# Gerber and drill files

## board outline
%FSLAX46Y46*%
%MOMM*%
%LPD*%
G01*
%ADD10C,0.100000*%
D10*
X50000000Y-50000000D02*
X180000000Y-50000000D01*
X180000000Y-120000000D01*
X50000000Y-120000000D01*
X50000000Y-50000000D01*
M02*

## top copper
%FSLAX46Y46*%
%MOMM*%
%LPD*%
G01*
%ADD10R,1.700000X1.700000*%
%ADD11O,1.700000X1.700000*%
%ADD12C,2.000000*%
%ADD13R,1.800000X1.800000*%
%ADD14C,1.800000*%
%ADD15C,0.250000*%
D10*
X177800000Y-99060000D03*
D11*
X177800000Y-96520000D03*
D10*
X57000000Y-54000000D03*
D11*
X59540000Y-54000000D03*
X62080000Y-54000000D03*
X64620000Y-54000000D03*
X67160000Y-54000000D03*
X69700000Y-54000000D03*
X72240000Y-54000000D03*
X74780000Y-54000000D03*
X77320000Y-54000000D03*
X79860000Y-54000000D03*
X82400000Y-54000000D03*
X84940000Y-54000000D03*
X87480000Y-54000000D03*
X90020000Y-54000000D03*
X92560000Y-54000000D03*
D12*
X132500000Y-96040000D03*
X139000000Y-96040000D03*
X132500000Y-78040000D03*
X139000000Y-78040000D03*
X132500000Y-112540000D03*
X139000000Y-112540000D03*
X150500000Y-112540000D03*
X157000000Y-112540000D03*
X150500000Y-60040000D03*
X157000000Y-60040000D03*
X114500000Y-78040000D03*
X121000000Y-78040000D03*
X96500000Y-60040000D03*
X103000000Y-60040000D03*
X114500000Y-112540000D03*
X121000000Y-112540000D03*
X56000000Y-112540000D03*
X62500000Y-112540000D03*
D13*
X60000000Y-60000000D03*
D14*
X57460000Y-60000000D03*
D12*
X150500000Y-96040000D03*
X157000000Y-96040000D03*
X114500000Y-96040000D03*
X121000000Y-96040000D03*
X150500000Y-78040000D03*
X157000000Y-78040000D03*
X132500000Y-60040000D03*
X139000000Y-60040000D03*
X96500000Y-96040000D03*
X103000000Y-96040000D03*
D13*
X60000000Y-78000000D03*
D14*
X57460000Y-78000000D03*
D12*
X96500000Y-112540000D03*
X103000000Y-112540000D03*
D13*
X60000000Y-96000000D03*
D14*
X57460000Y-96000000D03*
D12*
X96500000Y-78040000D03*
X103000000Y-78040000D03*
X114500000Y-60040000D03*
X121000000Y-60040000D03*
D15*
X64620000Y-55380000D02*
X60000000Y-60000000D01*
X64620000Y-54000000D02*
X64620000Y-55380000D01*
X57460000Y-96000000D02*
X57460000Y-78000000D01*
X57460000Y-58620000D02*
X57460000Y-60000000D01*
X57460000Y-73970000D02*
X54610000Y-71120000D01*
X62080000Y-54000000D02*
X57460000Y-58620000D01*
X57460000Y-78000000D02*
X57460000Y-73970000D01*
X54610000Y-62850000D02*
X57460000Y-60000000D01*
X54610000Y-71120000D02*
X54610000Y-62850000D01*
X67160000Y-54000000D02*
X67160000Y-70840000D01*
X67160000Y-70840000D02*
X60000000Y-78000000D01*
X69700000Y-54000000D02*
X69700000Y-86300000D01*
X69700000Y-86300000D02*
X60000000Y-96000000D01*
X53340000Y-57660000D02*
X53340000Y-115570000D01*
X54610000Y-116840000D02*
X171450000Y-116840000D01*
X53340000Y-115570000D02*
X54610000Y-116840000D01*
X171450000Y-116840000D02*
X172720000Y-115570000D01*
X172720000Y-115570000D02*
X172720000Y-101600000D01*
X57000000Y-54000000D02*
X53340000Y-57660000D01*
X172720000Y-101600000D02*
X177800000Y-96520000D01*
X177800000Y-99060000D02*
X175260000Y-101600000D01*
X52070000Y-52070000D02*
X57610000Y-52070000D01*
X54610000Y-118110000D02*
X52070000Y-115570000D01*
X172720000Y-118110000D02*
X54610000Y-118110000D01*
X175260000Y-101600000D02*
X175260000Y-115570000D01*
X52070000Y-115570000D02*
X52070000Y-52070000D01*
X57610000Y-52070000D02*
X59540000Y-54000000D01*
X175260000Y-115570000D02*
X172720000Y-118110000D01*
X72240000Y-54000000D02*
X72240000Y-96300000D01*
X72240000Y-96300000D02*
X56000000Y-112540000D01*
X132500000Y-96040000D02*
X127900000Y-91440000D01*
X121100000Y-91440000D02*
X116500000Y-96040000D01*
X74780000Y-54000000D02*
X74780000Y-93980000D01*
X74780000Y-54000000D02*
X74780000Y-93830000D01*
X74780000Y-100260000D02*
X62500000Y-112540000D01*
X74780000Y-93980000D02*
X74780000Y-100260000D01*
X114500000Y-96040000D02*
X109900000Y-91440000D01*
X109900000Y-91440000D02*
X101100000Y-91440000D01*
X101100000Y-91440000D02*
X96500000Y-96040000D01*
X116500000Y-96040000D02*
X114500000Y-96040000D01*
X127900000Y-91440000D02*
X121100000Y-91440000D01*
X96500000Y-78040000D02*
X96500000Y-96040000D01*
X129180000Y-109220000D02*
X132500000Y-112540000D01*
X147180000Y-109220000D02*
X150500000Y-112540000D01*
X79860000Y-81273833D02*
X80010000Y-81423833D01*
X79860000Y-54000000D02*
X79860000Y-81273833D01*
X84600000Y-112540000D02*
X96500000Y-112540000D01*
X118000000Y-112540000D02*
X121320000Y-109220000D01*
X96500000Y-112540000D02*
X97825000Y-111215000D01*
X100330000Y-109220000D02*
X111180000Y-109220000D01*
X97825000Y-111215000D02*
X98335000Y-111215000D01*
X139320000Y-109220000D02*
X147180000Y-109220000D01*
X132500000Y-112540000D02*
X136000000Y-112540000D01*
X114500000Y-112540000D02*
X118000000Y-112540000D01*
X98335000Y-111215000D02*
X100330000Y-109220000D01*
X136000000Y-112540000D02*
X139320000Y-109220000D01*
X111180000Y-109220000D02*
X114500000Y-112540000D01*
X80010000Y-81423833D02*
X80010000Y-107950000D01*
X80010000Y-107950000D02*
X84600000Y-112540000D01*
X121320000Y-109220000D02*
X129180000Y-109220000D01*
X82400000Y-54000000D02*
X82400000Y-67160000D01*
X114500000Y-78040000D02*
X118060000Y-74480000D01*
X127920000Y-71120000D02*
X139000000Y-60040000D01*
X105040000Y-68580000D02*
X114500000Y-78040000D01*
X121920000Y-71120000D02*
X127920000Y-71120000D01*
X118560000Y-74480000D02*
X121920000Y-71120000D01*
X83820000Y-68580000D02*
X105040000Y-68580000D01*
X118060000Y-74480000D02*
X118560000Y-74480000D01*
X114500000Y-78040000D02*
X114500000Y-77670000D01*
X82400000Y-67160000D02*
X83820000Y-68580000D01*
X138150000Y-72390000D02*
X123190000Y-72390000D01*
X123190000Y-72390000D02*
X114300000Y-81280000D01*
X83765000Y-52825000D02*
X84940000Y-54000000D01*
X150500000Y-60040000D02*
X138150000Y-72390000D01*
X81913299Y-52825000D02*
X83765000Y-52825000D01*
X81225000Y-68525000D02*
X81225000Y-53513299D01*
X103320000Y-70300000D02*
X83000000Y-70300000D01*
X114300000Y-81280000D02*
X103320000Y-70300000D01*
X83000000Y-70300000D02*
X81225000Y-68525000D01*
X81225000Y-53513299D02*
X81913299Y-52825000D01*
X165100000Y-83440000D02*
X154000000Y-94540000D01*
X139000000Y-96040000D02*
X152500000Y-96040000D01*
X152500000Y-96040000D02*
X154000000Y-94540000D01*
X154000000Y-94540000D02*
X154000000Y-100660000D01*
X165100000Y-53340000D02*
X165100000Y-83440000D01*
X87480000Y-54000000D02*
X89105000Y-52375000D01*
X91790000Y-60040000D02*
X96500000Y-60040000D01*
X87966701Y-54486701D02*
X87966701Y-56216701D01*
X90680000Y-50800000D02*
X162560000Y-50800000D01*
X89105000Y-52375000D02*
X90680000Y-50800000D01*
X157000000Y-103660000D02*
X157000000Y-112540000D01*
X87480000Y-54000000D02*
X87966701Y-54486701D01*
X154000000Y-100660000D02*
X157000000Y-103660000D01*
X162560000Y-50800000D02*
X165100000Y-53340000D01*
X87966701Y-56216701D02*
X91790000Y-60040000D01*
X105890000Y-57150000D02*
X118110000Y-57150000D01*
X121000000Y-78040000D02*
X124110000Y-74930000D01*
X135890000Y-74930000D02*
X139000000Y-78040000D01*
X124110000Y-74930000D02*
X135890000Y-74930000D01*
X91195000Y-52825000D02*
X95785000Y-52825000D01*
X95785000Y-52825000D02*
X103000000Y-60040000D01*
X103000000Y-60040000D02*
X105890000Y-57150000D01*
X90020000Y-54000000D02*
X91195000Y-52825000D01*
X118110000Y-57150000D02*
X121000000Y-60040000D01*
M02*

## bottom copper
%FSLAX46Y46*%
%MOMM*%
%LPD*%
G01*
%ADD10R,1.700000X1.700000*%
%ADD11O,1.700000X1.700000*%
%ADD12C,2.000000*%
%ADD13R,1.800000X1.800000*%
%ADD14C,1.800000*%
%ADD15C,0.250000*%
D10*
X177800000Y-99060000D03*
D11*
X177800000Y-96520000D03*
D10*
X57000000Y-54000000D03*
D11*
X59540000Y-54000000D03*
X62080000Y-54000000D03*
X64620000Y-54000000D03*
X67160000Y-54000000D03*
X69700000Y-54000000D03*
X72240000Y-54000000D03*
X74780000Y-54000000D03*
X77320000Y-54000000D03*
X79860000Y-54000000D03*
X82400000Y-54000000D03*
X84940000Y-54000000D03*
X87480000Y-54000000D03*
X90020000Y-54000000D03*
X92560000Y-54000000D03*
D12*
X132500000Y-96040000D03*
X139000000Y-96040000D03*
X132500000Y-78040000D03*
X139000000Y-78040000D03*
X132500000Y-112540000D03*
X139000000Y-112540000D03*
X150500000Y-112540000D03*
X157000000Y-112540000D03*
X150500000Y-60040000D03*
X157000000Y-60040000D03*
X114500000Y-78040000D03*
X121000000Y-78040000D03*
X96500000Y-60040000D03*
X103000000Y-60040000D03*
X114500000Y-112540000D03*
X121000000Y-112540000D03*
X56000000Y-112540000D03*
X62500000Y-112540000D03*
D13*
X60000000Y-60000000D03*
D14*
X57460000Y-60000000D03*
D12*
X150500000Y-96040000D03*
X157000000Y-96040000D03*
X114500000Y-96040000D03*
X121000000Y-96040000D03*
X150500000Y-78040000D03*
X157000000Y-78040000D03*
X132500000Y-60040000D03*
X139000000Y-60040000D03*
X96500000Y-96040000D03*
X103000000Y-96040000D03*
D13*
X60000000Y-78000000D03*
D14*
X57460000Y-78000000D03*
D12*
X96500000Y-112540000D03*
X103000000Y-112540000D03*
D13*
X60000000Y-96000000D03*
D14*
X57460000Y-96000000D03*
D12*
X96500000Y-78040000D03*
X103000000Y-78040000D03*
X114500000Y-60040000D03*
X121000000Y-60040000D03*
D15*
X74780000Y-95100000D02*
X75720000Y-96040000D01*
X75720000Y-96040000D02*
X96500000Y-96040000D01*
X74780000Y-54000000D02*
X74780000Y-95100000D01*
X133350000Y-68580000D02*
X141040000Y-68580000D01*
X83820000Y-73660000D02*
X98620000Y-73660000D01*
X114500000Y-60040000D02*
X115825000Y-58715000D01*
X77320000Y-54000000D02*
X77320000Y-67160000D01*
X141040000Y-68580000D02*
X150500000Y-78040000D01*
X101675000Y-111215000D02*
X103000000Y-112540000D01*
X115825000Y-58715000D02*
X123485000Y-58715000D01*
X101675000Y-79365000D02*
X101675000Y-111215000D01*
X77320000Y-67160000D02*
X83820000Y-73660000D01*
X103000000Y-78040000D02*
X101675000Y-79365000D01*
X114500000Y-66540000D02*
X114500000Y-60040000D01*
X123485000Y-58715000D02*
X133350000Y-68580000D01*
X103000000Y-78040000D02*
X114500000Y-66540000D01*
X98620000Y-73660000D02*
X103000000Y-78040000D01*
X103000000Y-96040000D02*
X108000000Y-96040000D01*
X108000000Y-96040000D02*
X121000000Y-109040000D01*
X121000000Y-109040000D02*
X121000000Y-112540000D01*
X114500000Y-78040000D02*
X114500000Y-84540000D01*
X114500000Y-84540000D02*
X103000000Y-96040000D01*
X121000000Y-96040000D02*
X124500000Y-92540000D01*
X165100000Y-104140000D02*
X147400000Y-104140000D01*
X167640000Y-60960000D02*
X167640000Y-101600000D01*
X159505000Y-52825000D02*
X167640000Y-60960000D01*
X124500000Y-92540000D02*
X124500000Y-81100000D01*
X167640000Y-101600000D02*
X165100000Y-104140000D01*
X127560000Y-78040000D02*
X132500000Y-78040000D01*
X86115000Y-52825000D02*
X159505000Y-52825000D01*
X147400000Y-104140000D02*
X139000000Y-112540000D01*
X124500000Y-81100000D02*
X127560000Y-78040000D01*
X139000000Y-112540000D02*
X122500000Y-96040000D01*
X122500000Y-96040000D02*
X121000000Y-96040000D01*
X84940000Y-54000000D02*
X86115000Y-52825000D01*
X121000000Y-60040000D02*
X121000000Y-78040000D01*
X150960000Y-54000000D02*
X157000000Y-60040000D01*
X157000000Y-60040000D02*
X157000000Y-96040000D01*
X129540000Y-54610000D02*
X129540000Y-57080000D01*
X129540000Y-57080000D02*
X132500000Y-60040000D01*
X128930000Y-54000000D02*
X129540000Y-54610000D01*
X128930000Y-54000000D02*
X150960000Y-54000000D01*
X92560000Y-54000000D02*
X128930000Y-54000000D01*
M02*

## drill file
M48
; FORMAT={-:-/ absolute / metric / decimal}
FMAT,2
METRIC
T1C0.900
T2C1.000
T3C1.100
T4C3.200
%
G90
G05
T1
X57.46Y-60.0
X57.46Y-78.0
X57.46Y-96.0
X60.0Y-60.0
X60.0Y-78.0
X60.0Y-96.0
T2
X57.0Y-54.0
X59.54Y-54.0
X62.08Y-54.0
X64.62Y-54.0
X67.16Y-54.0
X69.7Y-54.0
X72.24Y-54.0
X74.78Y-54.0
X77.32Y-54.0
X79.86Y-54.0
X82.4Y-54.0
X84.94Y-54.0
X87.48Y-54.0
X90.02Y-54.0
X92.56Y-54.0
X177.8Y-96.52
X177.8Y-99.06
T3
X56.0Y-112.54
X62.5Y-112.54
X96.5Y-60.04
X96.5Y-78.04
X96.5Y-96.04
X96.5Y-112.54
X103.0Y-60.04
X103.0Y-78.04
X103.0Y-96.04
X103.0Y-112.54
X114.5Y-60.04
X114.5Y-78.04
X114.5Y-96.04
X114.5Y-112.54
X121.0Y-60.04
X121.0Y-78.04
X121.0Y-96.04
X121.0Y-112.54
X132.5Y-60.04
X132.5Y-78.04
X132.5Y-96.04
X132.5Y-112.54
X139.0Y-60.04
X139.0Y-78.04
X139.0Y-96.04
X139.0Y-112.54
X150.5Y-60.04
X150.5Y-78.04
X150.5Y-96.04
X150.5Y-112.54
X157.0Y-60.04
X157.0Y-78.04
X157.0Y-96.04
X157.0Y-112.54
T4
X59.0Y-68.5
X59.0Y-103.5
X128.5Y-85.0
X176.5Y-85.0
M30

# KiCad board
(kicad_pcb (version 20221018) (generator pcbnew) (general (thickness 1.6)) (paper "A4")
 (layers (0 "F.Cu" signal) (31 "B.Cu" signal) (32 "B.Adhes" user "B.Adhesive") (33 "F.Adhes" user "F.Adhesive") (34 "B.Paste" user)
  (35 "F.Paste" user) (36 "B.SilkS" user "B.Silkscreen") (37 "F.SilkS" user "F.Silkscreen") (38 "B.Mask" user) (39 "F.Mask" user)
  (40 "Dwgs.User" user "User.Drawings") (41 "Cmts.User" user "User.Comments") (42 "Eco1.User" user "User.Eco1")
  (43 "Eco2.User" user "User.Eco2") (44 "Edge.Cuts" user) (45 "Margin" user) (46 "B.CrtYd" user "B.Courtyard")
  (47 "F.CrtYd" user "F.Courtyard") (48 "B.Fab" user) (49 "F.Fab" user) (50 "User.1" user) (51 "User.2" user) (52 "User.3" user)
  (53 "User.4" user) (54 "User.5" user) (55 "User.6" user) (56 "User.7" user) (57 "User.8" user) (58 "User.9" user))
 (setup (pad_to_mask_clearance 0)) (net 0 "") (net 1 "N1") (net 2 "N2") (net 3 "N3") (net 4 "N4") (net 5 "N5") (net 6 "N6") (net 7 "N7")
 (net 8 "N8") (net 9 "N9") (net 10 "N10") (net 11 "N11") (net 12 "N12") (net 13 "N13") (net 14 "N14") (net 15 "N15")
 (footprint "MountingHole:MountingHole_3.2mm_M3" (layer "F.Cu") (at 59 68.5)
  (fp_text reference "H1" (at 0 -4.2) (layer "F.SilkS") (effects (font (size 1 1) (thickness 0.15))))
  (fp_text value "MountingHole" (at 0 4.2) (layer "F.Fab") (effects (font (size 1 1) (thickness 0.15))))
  (pad "" np_thru_hole circle (at 0 0) (size 3.2 3.2) (drill 3.2) (layers "*.Cu" "*.Mask")))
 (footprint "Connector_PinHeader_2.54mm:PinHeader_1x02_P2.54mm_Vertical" (layer "F.Cu") (at 177.8 99.06 180)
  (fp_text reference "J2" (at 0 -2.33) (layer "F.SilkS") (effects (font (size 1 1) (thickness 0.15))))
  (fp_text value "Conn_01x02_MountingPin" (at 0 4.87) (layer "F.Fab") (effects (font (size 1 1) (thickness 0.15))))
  (pad "1" thru_hole rect (at 0 0 180) (size 1.7 1.7) (drill 1) (layers "*.Cu" "*.Mask") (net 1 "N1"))
  (pad "2" thru_hole oval (at 0 2.54 180) (size 1.7 1.7) (drill 1) (layers "*.Cu" "*.Mask") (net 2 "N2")))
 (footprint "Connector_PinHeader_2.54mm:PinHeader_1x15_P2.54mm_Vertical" (layer "F.Cu") (at 57 54 90)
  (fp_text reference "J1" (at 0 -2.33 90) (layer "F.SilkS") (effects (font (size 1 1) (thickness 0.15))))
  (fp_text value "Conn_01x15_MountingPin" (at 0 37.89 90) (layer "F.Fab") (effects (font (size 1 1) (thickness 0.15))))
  (pad "1" thru_hole rect (at 0 0 90) (size 1.7 1.7) (drill 1) (layers "*.Cu" "*.Mask") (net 2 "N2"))
  (pad "2" thru_hole oval (at 0 2.54 90) (size 1.7 1.7) (drill 1) (layers "*.Cu" "*.Mask") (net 1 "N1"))
  (pad "3" thru_hole oval (at 0 5.08 90) (size 1.7 1.7) (drill 1) (layers "*.Cu" "*.Mask") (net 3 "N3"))
  (pad "4" thru_hole oval (at 0 7.62 90) (size 1.7 1.7) (drill 1) (layers "*.Cu" "*.Mask") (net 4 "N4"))
  (pad "5" thru_hole oval (at 0 10.16 90) (size 1.7 1.7) (drill 1) (layers "*.Cu" "*.Mask") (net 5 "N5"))
  (pad "6" thru_hole oval (at 0 12.7 90) (size 1.7 1.7) (drill 1) (layers "*.Cu" "*.Mask") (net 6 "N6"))
  (pad "7" thru_hole oval (at 0 15.24 90) (size 1.7 1.7) (drill 1) (layers "*.Cu" "*.Mask") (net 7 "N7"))
  (pad "8" thru_hole oval (at 0 17.78 90) (size 1.7 1.7) (drill 1) (layers "*.Cu" "*.Mask") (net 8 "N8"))
  (pad "9" thru_hole oval (at 0 20.32 90) (size 1.7 1.7) (drill 1) (layers "*.Cu" "*.Mask") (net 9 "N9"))
  (pad "10" thru_hole oval (at 0 22.86 90) (size 1.7 1.7) (drill 1) (layers "*.Cu" "*.Mask") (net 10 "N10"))
  (pad "11" thru_hole oval (at 0 25.4 90) (size 1.7 1.7) (drill 1) (layers "*.Cu" "*.Mask") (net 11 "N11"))
  (pad "12" thru_hole oval (at 0 27.94 90) (size 1.7 1.7) (drill 1) (layers "*.Cu" "*.Mask") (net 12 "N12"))
  (pad "13" thru_hole oval (at 0 30.48 90) (size 1.7 1.7) (drill 1) (layers "*.Cu" "*.Mask") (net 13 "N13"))
  (pad "14" thru_hole oval (at 0 33.02 90) (size 1.7 1.7) (drill 1) (layers "*.Cu" "*.Mask") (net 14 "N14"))
  (pad "15" thru_hole oval (at 0 35.56 90) (size 1.7 1.7) (drill 1) (layers "*.Cu" "*.Mask") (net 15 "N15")))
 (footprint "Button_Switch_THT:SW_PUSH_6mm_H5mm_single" (layer "F.Cu") (at 132.5 93.5)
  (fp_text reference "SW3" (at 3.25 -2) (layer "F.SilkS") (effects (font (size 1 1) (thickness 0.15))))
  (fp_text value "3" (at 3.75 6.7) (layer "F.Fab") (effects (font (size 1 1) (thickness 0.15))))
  (pad "1" thru_hole circle (at 0 2.54 90) (size 2 2) (drill 1.1) (layers "*.Cu" "*.Mask") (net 8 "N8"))
  (pad "2" thru_hole circle (at 6.5 2.54 90) (size 2 2) (drill 1.1) (layers "*.Cu" "*.Mask") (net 13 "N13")))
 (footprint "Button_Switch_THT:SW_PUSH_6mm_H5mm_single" (layer "F.Cu") (at 132.5 75.5)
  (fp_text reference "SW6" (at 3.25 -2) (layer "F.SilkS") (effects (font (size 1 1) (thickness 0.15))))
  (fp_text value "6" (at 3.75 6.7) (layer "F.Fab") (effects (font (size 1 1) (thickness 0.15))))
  (pad "1" thru_hole circle (at 0 2.54 90) (size 2 2) (drill 1.1) (layers "*.Cu" "*.Mask") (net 12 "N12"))
  (pad "2" thru_hole circle (at 6.5 2.54 90) (size 2 2) (drill 1.1) (layers "*.Cu" "*.Mask") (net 14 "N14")))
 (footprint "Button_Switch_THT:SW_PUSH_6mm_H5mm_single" (layer "F.Cu") (at 132.5 110)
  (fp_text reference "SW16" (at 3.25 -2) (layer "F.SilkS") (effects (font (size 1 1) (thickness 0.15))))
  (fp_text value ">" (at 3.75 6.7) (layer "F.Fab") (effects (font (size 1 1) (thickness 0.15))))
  (pad "1" thru_hole circle (at 0 2.54 90) (size 2 2) (drill 1.1) (layers "*.Cu" "*.Mask") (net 10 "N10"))
  (pad "2" thru_hole circle (at 6.5 2.54 90) (size 2 2) (drill 1.1) (layers "*.Cu" "*.Mask") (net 12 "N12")))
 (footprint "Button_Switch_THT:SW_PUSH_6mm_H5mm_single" (layer "F.Cu") (at 150.5 110)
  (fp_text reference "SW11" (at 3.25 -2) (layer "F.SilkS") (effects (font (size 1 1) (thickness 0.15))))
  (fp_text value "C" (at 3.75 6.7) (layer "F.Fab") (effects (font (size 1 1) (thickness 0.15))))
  (pad "1" thru_hole circle (at 0 2.54 90) (size 2 2) (drill 1.1) (layers "*.Cu" "*.Mask") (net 10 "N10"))
  (pad "2" thru_hole circle (at 6.5 2.54 90) (size 2 2) (drill 1.1) (layers "*.Cu" "*.Mask") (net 13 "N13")))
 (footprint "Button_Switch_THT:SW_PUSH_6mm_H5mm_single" (layer "F.Cu") (at 150.5 57.5)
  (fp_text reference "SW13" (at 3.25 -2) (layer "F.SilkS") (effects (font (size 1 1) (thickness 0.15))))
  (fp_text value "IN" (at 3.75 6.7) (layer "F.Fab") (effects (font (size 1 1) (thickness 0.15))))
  (pad "1" thru_hole circle (at 0 2.54 90) (size 2 2) (drill 1.1) (layers "*.Cu" "*.Mask") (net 12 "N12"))
  (pad "2" thru_hole circle (at 6.5 2.54 90) (size 2 2) (drill 1.1) (layers "*.Cu" "*.Mask") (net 15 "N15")))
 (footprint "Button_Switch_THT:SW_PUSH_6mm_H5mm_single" (layer "F.Cu") (at 114.5 75.5)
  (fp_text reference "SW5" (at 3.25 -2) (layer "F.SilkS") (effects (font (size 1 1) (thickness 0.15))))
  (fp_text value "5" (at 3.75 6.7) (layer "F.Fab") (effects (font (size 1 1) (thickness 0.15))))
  (pad "1" thru_hole circle (at 0 2.54 90) (size 2 2) (drill 1.1) (layers "*.Cu" "*.Mask") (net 11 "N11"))
  (pad "2" thru_hole circle (at 6.5 2.54 90) (size 2 2) (drill 1.1) (layers "*.Cu" "*.Mask") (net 14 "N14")))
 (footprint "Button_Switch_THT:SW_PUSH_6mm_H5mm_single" (layer "F.Cu") (at 96.5 57.5)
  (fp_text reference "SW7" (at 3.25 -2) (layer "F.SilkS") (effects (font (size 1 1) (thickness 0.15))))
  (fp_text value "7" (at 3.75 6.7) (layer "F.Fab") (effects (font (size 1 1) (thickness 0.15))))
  (pad "1" thru_hole circle (at 0 2.54 90) (size 2 2) (drill 1.1) (layers "*.Cu" "*.Mask") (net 13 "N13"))
  (pad "2" thru_hole circle (at 6.5 2.54 90) (size 2 2) (drill 1.1) (layers "*.Cu" "*.Mask") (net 14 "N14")))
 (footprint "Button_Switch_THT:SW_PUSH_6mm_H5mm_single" (layer "F.Cu") (at 114.5 110)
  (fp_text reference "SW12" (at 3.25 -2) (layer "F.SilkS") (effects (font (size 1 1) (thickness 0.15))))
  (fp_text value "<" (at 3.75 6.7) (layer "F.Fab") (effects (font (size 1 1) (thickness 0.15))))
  (pad "1" thru_hole circle (at 0 2.54 90) (size 2 2) (drill 1.1) (layers "*.Cu" "*.Mask") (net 10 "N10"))
  (pad "2" thru_hole circle (at 6.5 2.54 90) (size 2 2) (drill 1.1) (layers "*.Cu" "*.Mask") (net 11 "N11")))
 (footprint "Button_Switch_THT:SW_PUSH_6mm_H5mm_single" (layer "F.Cu") (at 56 110)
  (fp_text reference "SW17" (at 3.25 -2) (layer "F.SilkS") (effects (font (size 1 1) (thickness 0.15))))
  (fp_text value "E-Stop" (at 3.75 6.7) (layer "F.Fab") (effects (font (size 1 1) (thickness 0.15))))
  (pad "1" thru_hole circle (at 0 2.54 90) (size 2 2) (drill 1.1) (layers "*.Cu" "*.Mask") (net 7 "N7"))
  (pad "2" thru_hole circle (at 6.5 2.54 90) (size 2 2) (drill 1.1) (layers "*.Cu" "*.Mask") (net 8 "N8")))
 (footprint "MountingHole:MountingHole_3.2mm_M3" (layer "F.Cu") (at 176.5 85)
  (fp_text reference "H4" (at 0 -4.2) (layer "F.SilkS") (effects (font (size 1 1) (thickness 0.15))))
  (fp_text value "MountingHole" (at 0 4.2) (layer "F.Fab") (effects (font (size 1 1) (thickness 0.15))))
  (pad "" np_thru_hole circle (at 0 0) (size 3.2 3.2) (drill 3.2) (layers "*.Cu" "*.Mask")))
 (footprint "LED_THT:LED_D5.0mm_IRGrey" (layer "F.Cu") (at 60 60 180)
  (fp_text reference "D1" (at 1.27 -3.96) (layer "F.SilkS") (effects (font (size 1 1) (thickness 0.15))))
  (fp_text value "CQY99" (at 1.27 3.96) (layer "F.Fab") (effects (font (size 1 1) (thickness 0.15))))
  (pad "1" thru_hole rect (at 0 0 180) (size 1.8 1.8) (drill 0.9) (layers "*.Cu" "*.Mask") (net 4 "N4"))
  (pad "2" thru_hole circle (at 2.54 0 180) (size 1.8 1.8) (drill 0.9) (layers "*.Cu" "*.Mask") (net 3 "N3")))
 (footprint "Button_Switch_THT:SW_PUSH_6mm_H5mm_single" (layer "F.Cu") (at 150.5 93.5)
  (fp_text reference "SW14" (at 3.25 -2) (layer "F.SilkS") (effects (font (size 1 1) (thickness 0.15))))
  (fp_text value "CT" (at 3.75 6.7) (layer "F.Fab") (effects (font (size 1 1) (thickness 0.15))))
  (pad "1" thru_hole circle (at 0 2.54 90) (size 2 2) (drill 1.1) (layers "*.Cu" "*.Mask") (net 13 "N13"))
  (pad "2" thru_hole circle (at 6.5 2.54 90) (size 2 2) (drill 1.1) (layers "*.Cu" "*.Mask") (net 15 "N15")))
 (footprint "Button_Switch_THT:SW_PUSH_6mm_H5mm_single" (layer "F.Cu") (at 114.5 93.5)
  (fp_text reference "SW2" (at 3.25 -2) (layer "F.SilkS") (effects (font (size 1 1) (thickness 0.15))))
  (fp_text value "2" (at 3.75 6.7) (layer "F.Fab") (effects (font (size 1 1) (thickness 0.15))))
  (pad "1" thru_hole circle (at 0 2.54 90) (size 2 2) (drill 1.1) (layers "*.Cu" "*.Mask") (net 8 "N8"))
  (pad "2" thru_hole circle (at 6.5 2.54 90) (size 2 2) (drill 1.1) (layers "*.Cu" "*.Mask") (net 12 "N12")))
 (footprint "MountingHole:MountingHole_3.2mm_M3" (layer "F.Cu") (at 128.5 85)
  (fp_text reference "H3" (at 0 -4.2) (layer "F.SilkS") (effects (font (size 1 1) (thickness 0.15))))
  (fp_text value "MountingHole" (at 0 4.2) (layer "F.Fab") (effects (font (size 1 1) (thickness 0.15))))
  (pad "" np_thru_hole circle (at 0 0) (size 3.2 3.2) (drill 3.2) (layers "*.Cu" "*.Mask")))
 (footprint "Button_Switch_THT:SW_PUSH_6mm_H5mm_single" (layer "F.Cu") (at 150.5 75.5)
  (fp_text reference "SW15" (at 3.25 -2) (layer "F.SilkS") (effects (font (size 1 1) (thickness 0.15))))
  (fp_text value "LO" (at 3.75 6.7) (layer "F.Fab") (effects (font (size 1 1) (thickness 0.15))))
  (pad "1" thru_hole circle (at 0 2.54 90) (size 2 2) (drill 1.1) (layers "*.Cu" "*.Mask") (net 9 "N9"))
  (pad "2" thru_hole circle (at 6.5 2.54 90) (size 2 2) (drill 1.1) (layers "*.Cu" "*.Mask") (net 15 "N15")))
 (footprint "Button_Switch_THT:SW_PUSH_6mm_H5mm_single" (layer "F.Cu") (at 132.5 57.5)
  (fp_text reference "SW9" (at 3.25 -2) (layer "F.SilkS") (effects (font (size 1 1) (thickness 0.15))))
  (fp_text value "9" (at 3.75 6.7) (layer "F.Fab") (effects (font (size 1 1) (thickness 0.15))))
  (pad "1" thru_hole circle (at 0 2.54 90) (size 2 2) (drill 1.1) (layers "*.Cu" "*.Mask") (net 15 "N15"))
  (pad "2" thru_hole circle (at 6.5 2.54 90) (size 2 2) (drill 1.1) (layers "*.Cu" "*.Mask") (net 11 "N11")))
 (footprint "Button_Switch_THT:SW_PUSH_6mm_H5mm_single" (layer "F.Cu") (at 96.5 93.5)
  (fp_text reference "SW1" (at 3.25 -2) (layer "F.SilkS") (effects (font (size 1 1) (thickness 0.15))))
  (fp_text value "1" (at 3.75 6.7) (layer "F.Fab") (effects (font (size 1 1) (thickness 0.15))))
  (pad "1" thru_hole circle (at 0 2.54 90) (size 2 2) (drill 1.1) (layers "*.Cu" "*.Mask") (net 8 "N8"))
  (pad "2" thru_hole circle (at 6.5 2.54 90) (size 2 2) (drill 1.1) (layers "*.Cu" "*.Mask") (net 11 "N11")))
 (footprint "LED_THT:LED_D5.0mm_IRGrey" (layer "F.Cu") (at 60 78 180)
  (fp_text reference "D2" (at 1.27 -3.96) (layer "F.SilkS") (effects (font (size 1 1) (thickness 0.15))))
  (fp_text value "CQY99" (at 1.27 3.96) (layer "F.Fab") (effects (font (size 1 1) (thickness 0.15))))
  (pad "1" thru_hole rect (at 0 0 180) (size 1.8 1.8) (drill 0.9) (layers "*.Cu" "*.Mask") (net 5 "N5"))
  (pad "2" thru_hole circle (at 2.54 0 180) (size 1.8 1.8) (drill 0.9) (layers "*.Cu" "*.Mask") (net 3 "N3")))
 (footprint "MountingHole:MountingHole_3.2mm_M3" (layer "F.Cu") (at 59 103.5)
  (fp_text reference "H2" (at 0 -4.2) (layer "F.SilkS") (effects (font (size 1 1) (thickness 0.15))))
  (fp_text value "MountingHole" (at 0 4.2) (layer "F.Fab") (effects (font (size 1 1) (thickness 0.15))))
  (pad "" np_thru_hole circle (at 0 0) (size 3.2 3.2) (drill 3.2) (layers "F&B.Cu" "*.Mask")))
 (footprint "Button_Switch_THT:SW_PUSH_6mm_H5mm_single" (layer "F.Cu") (at 96.5 110)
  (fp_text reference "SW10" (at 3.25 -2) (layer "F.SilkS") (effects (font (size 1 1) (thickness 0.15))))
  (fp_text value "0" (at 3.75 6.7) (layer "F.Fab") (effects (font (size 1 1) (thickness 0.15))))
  (pad "1" thru_hole circle (at 0 2.54 90) (size 2 2) (drill 1.1) (layers "*.Cu" "*.Mask") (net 10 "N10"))
  (pad "2" thru_hole circle (at 6.5 2.54 90) (size 2 2) (drill 1.1) (layers "*.Cu" "*.Mask") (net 9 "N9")))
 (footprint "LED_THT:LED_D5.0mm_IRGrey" (layer "F.Cu") (at 60 96 180)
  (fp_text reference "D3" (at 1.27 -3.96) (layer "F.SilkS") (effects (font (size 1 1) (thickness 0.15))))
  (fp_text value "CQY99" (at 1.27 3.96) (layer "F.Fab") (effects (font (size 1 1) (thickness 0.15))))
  (pad "1" thru_hole rect (at 0 0 180) (size 1.8 1.8) (drill 0.9) (layers "*.Cu" "*.Mask") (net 6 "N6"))
  (pad "2" thru_hole circle (at 2.54 0 180) (size 1.8 1.8) (drill 0.9) (layers "*.Cu" "*.Mask") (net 3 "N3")))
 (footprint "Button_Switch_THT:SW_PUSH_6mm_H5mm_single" (layer "F.Cu") (at 96.5 75.5)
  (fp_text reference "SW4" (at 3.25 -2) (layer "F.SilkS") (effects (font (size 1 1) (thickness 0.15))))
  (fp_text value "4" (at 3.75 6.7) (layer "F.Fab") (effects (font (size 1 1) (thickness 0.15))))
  (pad "1" thru_hole circle (at 0 2.54 90) (size 2 2) (drill 1.1) (layers "*.Cu" "*.Mask") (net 8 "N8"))
  (pad "2" thru_hole circle (at 6.5 2.54 90) (size 2 2) (drill 1.1) (layers "*.Cu" "*.Mask") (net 9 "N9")))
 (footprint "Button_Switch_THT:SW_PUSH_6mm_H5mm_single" (layer "F.Cu") (at 114.5 57.5)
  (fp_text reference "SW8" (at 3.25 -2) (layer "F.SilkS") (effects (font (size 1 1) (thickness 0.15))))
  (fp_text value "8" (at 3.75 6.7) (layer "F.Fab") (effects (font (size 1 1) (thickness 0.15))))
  (pad "1" thru_hole circle (at 0 2.54 90) (size 2 2) (drill 1.1) (layers "*.Cu" "*.Mask") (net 9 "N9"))
  (pad "2" thru_hole circle (at 6.5 2.54 90) (size 2 2) (drill 1.1) (layers "*.Cu" "*.Mask") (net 14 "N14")))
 (gr_rect (start 50 50) (end 180 120) (stroke (width 0.1) (type default)) (fill none) (layer "Edge.Cuts"))
 (segment (start 64.62 55.38) (end 60 60) (width 0.25) (layer "F.Cu") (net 4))
 (segment (start 64.62 54) (end 64.62 55.38) (width 0.25) (layer "F.Cu") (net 4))
 (segment (start 57.46 96) (end 57.46 78) (width 0.25) (layer "F.Cu") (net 3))
 (segment (start 57.46 58.62) (end 57.46 60) (width 0.25) (layer "F.Cu") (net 3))
 (segment (start 57.46 73.97) (end 54.61 71.12) (width 0.25) (layer "F.Cu") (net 3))
 (segment (start 62.08 54) (end 57.46 58.62) (width 0.25) (layer "F.Cu") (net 3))
 (segment (start 57.46 78) (end 57.46 73.97) (width 0.25) (layer "F.Cu") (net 3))
 (segment (start 54.61 62.85) (end 57.46 60) (width 0.25) (layer "F.Cu") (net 3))
 (segment (start 54.61 71.12) (end 54.61 62.85) (width 0.25) (layer "F.Cu") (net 3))
 (segment (start 67.16 54) (end 67.16 70.84) (width 0.25) (layer "F.Cu") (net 5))
 (segment (start 67.16 70.84) (end 60 78) (width 0.25) (layer "F.Cu") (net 5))
 (segment (start 69.7 54) (end 69.7 86.3) (width 0.25) (layer "F.Cu") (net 6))
 (segment (start 69.7 86.3) (end 60 96) (width 0.25) (layer "F.Cu") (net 6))
 (segment (start 53.34 57.66) (end 53.34 115.57) (width 0.25) (layer "F.Cu") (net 2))
 (segment (start 54.61 116.84) (end 171.45 116.84) (width 0.25) (layer "F.Cu") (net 2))
 (segment (start 53.34 115.57) (end 54.61 116.84) (width 0.25) (layer "F.Cu") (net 2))
 (segment (start 171.45 116.84) (end 172.72 115.57) (width 0.25) (layer "F.Cu") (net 2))
 (segment (start 172.72 115.57) (end 172.72 101.6) (width 0.25) (layer "F.Cu") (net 2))
 (segment (start 57 54) (end 53.34 57.66) (width 0.25) (layer "F.Cu") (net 2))
 (segment (start 172.72 101.6) (end 177.8 96.52) (width 0.25) (layer "F.Cu") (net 2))
 (segment (start 177.8 99.06) (end 175.26 101.6) (width 0.25) (layer "F.Cu") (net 1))
 (segment (start 52.07 52.07) (end 57.61 52.07) (width 0.25) (layer "F.Cu") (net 1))
 (segment (start 54.61 118.11) (end 52.07 115.57) (width 0.25) (layer "F.Cu") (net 1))
 (segment (start 172.72 118.11) (end 54.61 118.11) (width 0.25) (layer "F.Cu") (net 1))
 (segment (start 175.26 101.6) (end 175.26 115.57) (width 0.25) (layer "F.Cu") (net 1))
 (segment (start 52.07 115.57) (end 52.07 52.07) (width 0.25) (layer "F.Cu") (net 1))
 (segment (start 57.61 52.07) (end 59.54 54) (width 0.25) (layer "F.Cu") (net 1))
 (segment (start 175.26 115.57) (end 172.72 118.11) (width 0.25) (layer "F.Cu") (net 1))
 (segment (start 72.24 54) (end 72.24 96.3) (width 0.25) (layer "F.Cu") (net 7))
 (segment (start 72.24 96.3) (end 56 112.54) (width 0.25) (layer "F.Cu") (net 7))
 (segment (start 132.5 96.04) (end 127.9 91.44) (width 0.25) (layer "F.Cu") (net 8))
 (segment (start 121.1 91.44) (end 116.5 96.04) (width 0.25) (layer "F.Cu") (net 8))
 (segment (start 74.78 54) (end 74.78 93.98) (width 0.25) (layer "F.Cu") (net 8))
 (segment (start 74.78 54) (end 74.78 93.83) (width 0.25) (layer "F.Cu") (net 8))
 (segment (start 74.78 100.26) (end 62.5 112.54) (width 0.25) (layer "F.Cu") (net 8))
 (segment (start 74.78 93.98) (end 74.78 100.26) (width 0.25) (layer "F.Cu") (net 8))
 (segment (start 114.5 96.04) (end 109.9 91.44) (width 0.25) (layer "F.Cu") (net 8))
 (segment (start 109.9 91.44) (end 101.1 91.44) (width 0.25) (layer "F.Cu") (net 8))
 (segment (start 101.1 91.44) (end 96.5 96.04) (width 0.25) (layer "F.Cu") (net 8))
 (segment (start 116.5 96.04) (end 114.5 96.04) (width 0.25) (layer "F.Cu") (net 8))
 (segment (start 127.9 91.44) (end 121.1 91.44) (width 0.25) (layer "F.Cu") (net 8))
 (segment (start 96.5 78.04) (end 96.5 96.04) (width 0.25) (layer "F.Cu") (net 8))
 (segment (start 74.78 95.1) (end 75.72 96.04) (width 0.25) (layer "B.Cu") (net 8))
 (segment (start 75.72 96.04) (end 96.5 96.04) (width 0.25) (layer "B.Cu") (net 8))
 (segment (start 74.78 54) (end 74.78 95.1) (width 0.25) (layer "B.Cu") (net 8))
 (segment (start 133.35 68.58) (end 141.04 68.58) (width 0.25) (layer "B.Cu") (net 9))
 (segment (start 83.82 73.66) (end 98.62 73.66) (width 0.25) (layer "B.Cu") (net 9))
 (segment (start 114.5 60.04) (end 115.825 58.715) (width 0.25) (layer "B.Cu") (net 9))
 (segment (start 77.32 54) (end 77.32 67.16) (width 0.25) (layer "B.Cu") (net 9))
 (segment (start 141.04 68.58) (end 150.5 78.04) (width 0.25) (layer "B.Cu") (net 9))
 (segment (start 101.675 111.215) (end 103 112.54) (width 0.25) (layer "B.Cu") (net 9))
 (segment (start 115.825 58.715) (end 123.485 58.715) (width 0.25) (layer "B.Cu") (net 9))
 (segment (start 101.675 79.365) (end 101.675 111.215) (width 0.25) (layer "B.Cu") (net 9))
 (segment (start 77.32 67.16) (end 83.82 73.66) (width 0.25) (layer "B.Cu") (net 9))
 (segment (start 103 78.04) (end 101.675 79.365) (width 0.25) (layer "B.Cu") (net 9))
 (segment (start 114.5 66.54) (end 114.5 60.04) (width 0.25) (layer "B.Cu") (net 9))
 (segment (start 123.485 58.715) (end 133.35 68.58) (width 0.25) (layer "B.Cu") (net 9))
 (segment (start 103 78.04) (end 114.5 66.54) (width 0.25) (layer "B.Cu") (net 9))
 (segment (start 98.62 73.66) (end 103 78.04) (width 0.25) (layer "B.Cu") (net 9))
 (segment (start 129.18 109.22) (end 132.5 112.54) (width 0.25) (layer "F.Cu") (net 10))
 (segment (start 147.18 109.22) (end 150.5 112.54) (width 0.25) (layer "F.Cu") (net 10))
 (segment (start 79.86 81.273833) (end 80.01 81.423833) (width 0.25) (layer "F.Cu") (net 10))
 (segment (start 79.86 54) (end 79.86 81.273833) (width 0.25) (layer "F.Cu") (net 10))
 (segment (start 84.6 112.54) (end 96.5 112.54) (width 0.25) (layer "F.Cu") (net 10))
 (segment (start 118 112.54) (end 121.32 109.22) (width 0.25) (layer "F.Cu") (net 10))
 (segment (start 96.5 112.54) (end 97.825 111.215) (width 0.25) (layer "F.Cu") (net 10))
 (segment (start 100.33 109.22) (end 111.18 109.22) (width 0.25) (layer "F.Cu") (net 10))
 (segment (start 97.825 111.215) (end 98.335 111.215) (width 0.25) (layer "F.Cu") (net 10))
 (segment (start 139.32 109.22) (end 147.18 109.22) (width 0.25) (layer "F.Cu") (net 10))
 (segment (start 132.5 112.54) (end 136 112.54) (width 0.25) (layer "F.Cu") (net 10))
 (segment (start 114.5 112.54) (end 118 112.54) (width 0.25) (layer "F.Cu") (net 10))
 (segment (start 98.335 111.215) (end 100.33 109.22) (width 0.25) (layer "F.Cu") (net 10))
 (segment (start 136 112.54) (end 139.32 109.22) (width 0.25) (layer "F.Cu") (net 10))
 (segment (start 111.18 109.22) (end 114.5 112.54) (width 0.25) (layer "F.Cu") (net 10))
 (segment (start 80.01 81.423833) (end 80.01 107.95) (width 0.25) (layer "F.Cu") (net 10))
 (segment (start 80.01 107.95) (end 84.6 112.54) (width 0.25) (layer "F.Cu") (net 10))
 (segment (start 121.32 109.22) (end 129.18 109.22) (width 0.25) (layer "F.Cu") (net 10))
 (segment (start 82.4 54) (end 82.4 67.16) (width 0.25) (layer "F.Cu") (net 11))
 (segment (start 114.5 78.04) (end 118.06 74.48) (width 0.25) (layer "F.Cu") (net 11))
 (segment (start 127.92 71.12) (end 139 60.04) (width 0.25) (layer "F.Cu") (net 11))
 (segment (start 105.04 68.58) (end 114.5 78.04) (width 0.25) (layer "F.Cu") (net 11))
 (segment (start 121.92 71.12) (end 127.92 71.12) (width 0.25) (layer "F.Cu") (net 11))
 (segment (start 118.56 74.48) (end 121.92 71.12) (width 0.25) (layer "F.Cu") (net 11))
 (segment (start 83.82 68.58) (end 105.04 68.58) (width 0.25) (layer "F.Cu") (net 11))
 (segment (start 118.06 74.48) (end 118.56 74.48) (width 0.25) (layer "F.Cu") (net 11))
 (segment (start 114.5 78.04) (end 114.5 77.67) (width 0.25) (layer "F.Cu") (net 11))
 (segment (start 82.4 67.16) (end 83.82 68.58) (width 0.25) (layer "F.Cu") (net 11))
 (segment (start 103 96.04) (end 108 96.04) (width 0.25) (layer "B.Cu") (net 11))
 (segment (start 108 96.04) (end 121 109.04) (width 0.25) (layer "B.Cu") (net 11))
 (segment (start 121 109.04) (end 121 112.54) (width 0.25) (layer "B.Cu") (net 11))
 (segment (start 114.5 78.04) (end 114.5 84.54) (width 0.25) (layer "B.Cu") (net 11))
 (segment (start 114.5 84.54) (end 103 96.04) (width 0.25) (layer "B.Cu") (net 11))
 (segment (start 138.15 72.39) (end 123.19 72.39) (width 0.25) (layer "F.Cu") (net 12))
 (segment (start 123.19 72.39) (end 114.3 81.28) (width 0.25) (layer "F.Cu") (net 12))
 (segment (start 83.765 52.825) (end 84.94 54) (width 0.25) (layer "F.Cu") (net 12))
 (segment (start 150.5 60.04) (end 138.15 72.39) (width 0.25) (layer "F.Cu") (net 12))
 (segment (start 81.913299 52.825) (end 83.765 52.825) (width 0.25) (layer "F.Cu") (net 12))
 (segment (start 81.225 68.525) (end 81.225 53.513299) (width 0.25) (layer "F.Cu") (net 12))
 (segment (start 103.32 70.3) (end 83 70.3) (width 0.25) (layer "F.Cu") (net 12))
 (segment (start 114.3 81.28) (end 103.32 70.3) (width 0.25) (layer "F.Cu") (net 12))
 (segment (start 83 70.3) (end 81.225 68.525) (width 0.25) (layer "F.Cu") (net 12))
 (segment (start 81.225 53.513299) (end 81.913299 52.825) (width 0.25) (layer "F.Cu") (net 12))
 (segment (start 121 96.04) (end 124.5 92.54) (width 0.25) (layer "B.Cu") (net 12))
 (segment (start 165.1 104.14) (end 147.4 104.14) (width 0.25) (layer "B.Cu") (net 12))
 (segment (start 167.64 60.96) (end 167.64 101.6) (width 0.25) (layer "B.Cu") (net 12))
 (segment (start 159.505 52.825) (end 167.64 60.96) (width 0.25) (layer "B.Cu") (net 12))
 (segment (start 124.5 92.54) (end 124.5 81.1) (width 0.25) (layer "B.Cu") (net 12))
 (segment (start 167.64 101.6) (end 165.1 104.14) (width 0.25) (layer "B.Cu") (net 12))
 (segment (start 127.56 78.04) (end 132.5 78.04) (width 0.25) (layer "B.Cu") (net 12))
 (segment (start 86.115 52.825) (end 159.505 52.825) (width 0.25) (layer "B.Cu") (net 12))
 (segment (start 147.4 104.14) (end 139 112.54) (width 0.25) (layer "B.Cu") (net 12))
 (segment (start 124.5 81.1) (end 127.56 78.04) (width 0.25) (layer "B.Cu") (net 12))
 (segment (start 139 112.54) (end 122.5 96.04) (width 0.25) (layer "B.Cu") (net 12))
 (segment (start 122.5 96.04) (end 121 96.04) (width 0.25) (layer "B.Cu") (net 12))
 (segment (start 84.94 54) (end 86.115 52.825) (width 0.25) (layer "B.Cu") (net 12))
 (segment (start 165.1 83.44) (end 154 94.54) (width 0.25) (layer "F.Cu") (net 13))
 (segment (start 139 96.04) (end 152.5 96.04) (width 0.25) (layer "F.Cu") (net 13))
 (segment (start 152.5 96.04) (end 154 94.54) (width 0.25) (layer "F.Cu") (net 13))
 (segment (start 154 94.54) (end 154 100.66) (width 0.25) (layer "F.Cu") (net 13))
 (segment (start 165.1 53.34) (end 165.1 83.44) (width 0.25) (layer "F.Cu") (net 13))
 (segment (start 87.48 54) (end 89.105 52.375) (width 0.25) (layer "F.Cu") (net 13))
 (segment (start 91.79 60.04) (end 96.5 60.04) (width 0.25) (layer "F.Cu") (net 13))
 (segment (start 87.966701 54.486701) (end 87.966701 56.216701) (width 0.25) (layer "F.Cu") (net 13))
 (segment (start 90.68 50.8) (end 162.56 50.8) (width 0.25) (layer "F.Cu") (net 13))
 (segment (start 89.105 52.375) (end 90.68 50.8) (width 0.25) (layer "F.Cu") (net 13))
 (segment (start 157 103.66) (end 157 112.54) (width 0.25) (layer "F.Cu") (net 13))
 (segment (start 87.48 54) (end 87.966701 54.486701) (width 0.25) (layer "F.Cu") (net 13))
 (segment (start 154 100.66) (end 157 103.66) (width 0.25) (layer "F.Cu") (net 13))
 (segment (start 162.56 50.8) (end 165.1 53.34) (width 0.25) (layer "F.Cu") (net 13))
 (segment (start 87.966701 56.216701) (end 91.79 60.04) (width 0.25) (layer "F.Cu") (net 13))
 (segment (start 105.89 57.15) (end 118.11 57.15) (width 0.25) (layer "F.Cu") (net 14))
 (segment (start 121 78.04) (end 124.11 74.93) (width 0.25) (layer "F.Cu") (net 14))
 (segment (start 135.89 74.93) (end 139 78.04) (width 0.25) (layer "F.Cu") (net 14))
 (segment (start 124.11 74.93) (end 135.89 74.93) (width 0.25) (layer "F.Cu") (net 14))
 (segment (start 91.195 52.825) (end 95.785 52.825) (width 0.25) (layer "F.Cu") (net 14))
 (segment (start 95.785 52.825) (end 103 60.04) (width 0.25) (layer "F.Cu") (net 14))
 (segment (start 103 60.04) (end 105.89 57.15) (width 0.25) (layer "F.Cu") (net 14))
 (segment (start 90.02 54) (end 91.195 52.825) (width 0.25) (layer "F.Cu") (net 14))
 (segment (start 118.11 57.15) (end 121 60.04) (width 0.25) (layer "F.Cu") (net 14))
 (segment (start 121 60.04) (end 121 78.04) (width 0.25) (layer "B.Cu") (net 14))
 (segment (start 150.96 54) (end 157 60.04) (width 0.25) (layer "B.Cu") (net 15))
 (segment (start 157 60.04) (end 157 96.04) (width 0.25) (layer "B.Cu") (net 15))
 (segment (start 129.54 54.61) (end 129.54 57.08) (width 0.25) (layer "B.Cu") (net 15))
 (segment (start 129.54 57.08) (end 132.5 60.04) (width 0.25) (layer "B.Cu") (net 15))
 (segment (start 128.93 54) (end 129.54 54.61) (width 0.25) (layer "B.Cu") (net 15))
 (segment (start 128.93 54) (end 150.96 54) (width 0.25) (layer "B.Cu") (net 15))
 (segment (start 92.56 54) (end 128.93 54) (width 0.25) (layer "B.Cu") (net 15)))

